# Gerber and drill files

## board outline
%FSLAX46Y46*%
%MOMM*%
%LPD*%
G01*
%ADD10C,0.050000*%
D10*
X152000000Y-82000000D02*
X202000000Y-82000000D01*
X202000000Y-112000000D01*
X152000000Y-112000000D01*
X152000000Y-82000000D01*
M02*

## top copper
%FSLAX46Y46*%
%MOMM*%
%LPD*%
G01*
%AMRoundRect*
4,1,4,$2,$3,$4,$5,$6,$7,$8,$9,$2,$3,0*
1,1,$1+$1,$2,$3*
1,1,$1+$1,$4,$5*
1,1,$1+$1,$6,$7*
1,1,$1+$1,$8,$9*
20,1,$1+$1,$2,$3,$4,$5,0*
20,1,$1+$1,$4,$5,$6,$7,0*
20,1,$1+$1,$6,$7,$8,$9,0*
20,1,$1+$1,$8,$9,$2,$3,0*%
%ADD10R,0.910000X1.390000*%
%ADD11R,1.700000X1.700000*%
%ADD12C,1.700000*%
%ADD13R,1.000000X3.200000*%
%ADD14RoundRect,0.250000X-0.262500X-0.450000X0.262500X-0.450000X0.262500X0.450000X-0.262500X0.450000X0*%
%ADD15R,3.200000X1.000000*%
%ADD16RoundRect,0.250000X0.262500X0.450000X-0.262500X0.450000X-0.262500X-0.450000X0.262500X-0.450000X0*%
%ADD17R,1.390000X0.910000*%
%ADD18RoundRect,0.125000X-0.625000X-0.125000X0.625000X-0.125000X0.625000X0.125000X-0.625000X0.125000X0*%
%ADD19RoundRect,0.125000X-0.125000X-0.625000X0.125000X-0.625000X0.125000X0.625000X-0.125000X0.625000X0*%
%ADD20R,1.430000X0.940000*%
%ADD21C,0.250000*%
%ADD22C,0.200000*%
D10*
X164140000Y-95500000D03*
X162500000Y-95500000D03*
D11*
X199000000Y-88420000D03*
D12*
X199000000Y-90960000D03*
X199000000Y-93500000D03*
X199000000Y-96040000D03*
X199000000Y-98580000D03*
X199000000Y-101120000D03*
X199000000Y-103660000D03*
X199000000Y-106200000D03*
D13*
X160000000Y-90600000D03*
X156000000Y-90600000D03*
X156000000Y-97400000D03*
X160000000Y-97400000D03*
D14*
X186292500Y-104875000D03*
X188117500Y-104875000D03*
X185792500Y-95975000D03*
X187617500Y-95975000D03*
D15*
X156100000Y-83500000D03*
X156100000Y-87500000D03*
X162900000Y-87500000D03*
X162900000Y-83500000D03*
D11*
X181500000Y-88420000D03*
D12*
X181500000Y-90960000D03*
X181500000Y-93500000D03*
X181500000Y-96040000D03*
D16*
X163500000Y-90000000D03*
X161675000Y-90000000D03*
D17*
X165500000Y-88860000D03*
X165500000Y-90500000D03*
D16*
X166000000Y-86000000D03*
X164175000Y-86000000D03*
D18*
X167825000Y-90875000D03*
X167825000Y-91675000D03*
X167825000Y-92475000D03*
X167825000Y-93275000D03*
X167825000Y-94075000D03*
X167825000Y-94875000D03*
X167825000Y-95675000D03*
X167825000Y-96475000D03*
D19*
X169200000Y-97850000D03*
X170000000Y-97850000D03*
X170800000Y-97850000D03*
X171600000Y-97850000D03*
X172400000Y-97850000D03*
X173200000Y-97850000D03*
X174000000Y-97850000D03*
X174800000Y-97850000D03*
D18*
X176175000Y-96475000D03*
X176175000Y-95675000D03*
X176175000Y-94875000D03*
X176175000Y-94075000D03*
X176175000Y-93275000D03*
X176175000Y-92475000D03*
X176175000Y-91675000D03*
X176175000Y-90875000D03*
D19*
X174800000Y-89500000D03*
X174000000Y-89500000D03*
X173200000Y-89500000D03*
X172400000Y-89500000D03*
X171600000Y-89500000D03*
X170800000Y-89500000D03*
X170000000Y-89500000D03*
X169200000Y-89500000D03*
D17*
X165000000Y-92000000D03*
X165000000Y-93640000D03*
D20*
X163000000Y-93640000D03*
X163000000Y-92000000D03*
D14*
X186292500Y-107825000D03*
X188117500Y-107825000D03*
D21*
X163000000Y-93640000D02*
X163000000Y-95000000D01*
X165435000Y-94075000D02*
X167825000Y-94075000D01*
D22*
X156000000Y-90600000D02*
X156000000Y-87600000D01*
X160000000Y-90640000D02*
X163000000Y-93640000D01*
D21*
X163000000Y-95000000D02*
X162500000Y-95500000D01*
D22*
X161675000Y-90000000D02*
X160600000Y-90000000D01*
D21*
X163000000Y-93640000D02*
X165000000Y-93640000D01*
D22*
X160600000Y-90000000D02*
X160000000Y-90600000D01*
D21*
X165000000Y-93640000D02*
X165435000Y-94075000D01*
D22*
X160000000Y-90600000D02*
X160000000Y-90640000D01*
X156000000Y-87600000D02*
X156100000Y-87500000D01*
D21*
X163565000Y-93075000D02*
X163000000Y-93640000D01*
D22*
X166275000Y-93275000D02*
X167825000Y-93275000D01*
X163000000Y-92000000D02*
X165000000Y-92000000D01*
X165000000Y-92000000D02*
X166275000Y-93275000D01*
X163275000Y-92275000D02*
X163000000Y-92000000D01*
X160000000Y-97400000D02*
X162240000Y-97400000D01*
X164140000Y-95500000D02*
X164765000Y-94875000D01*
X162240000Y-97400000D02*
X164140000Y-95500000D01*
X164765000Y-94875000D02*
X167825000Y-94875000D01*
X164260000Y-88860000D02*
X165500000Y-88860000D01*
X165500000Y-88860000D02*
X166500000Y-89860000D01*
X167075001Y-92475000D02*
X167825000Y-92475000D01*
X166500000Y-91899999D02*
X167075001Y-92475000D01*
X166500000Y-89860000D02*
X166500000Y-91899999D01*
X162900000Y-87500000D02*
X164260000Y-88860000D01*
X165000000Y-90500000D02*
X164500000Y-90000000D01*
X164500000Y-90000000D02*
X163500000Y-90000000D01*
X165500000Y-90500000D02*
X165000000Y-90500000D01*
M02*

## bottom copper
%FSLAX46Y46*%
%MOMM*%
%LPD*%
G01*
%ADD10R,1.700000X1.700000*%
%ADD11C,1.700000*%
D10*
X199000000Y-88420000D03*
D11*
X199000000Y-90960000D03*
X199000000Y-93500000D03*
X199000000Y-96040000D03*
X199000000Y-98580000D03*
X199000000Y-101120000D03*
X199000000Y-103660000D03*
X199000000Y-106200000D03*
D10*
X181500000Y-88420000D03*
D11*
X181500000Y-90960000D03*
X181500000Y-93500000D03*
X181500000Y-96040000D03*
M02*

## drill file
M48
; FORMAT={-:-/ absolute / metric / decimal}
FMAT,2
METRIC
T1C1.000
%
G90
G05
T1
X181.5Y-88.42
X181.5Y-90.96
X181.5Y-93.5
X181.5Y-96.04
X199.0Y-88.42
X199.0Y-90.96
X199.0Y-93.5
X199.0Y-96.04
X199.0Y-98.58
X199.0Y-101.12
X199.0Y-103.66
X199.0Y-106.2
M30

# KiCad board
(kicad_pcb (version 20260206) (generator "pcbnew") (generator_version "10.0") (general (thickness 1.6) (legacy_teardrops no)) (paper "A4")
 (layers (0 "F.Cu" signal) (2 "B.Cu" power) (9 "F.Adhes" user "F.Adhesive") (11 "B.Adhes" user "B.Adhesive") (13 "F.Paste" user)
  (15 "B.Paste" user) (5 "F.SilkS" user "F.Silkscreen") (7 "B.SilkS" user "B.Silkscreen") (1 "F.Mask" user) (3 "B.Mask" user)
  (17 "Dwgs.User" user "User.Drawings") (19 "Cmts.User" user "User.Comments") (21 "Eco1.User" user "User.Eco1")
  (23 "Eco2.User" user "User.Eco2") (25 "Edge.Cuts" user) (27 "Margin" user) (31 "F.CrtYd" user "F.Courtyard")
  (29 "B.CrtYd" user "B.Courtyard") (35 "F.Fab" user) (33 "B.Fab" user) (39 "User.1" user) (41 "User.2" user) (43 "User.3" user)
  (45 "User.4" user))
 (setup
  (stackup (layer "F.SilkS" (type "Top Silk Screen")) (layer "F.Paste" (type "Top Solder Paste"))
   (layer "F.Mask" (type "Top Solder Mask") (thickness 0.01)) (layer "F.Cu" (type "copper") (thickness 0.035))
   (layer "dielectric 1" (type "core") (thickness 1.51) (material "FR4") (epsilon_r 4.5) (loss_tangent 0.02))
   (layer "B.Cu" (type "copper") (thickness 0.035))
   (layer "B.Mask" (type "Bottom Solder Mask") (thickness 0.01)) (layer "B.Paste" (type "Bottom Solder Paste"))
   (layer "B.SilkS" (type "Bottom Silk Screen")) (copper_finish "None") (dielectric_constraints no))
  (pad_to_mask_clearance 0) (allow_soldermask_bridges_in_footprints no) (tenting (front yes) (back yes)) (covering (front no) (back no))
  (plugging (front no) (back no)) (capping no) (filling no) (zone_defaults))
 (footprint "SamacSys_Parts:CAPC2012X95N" (layer "F.Cu") (at 163.32 95.5 180)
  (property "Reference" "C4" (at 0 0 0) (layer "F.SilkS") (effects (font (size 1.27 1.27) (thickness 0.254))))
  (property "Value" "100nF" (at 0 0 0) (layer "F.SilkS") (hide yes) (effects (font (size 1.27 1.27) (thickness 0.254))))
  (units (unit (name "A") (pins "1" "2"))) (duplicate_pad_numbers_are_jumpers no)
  (pad "1" smd rect (at -0.82 0 180) (size 0.91 1.39) (layers "F.Cu" "F.Mask" "F.Paste") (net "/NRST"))
  (pad "2" smd rect (at 0.82 0 180) (size 0.91 1.39) (layers "F.Cu" "F.Mask" "F.Paste") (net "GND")))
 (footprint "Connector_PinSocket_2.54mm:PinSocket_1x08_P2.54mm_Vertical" (layer "F.Cu") (at 199 88.42)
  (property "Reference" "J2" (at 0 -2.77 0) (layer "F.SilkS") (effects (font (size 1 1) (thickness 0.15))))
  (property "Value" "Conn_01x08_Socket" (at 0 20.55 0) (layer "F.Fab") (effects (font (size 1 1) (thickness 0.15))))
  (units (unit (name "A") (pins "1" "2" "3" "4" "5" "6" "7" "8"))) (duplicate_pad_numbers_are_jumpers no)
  (pad "1" thru_hole rect (at 0 0) (size 1.7 1.7) (drill 1) (layers "*.Cu" "*.Mask") (remove_unused_layers no) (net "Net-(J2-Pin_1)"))
  (pad "2" thru_hole circle (at 0 2.54) (size 1.7 1.7) (drill 1) (layers "*.Cu" "*.Mask") (remove_unused_layers no)
   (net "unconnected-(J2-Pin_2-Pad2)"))
  (pad "3" thru_hole circle (at 0 5.08) (size 1.7 1.7) (drill 1) (layers "*.Cu" "*.Mask") (remove_unused_layers no)
   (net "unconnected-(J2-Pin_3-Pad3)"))
  (pad "4" thru_hole circle (at 0 7.62) (size 1.7 1.7) (drill 1) (layers "*.Cu" "*.Mask") (remove_unused_layers no)
   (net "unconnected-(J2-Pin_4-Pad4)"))
  (pad "5" thru_hole circle (at 0 10.16) (size 1.7 1.7) (drill 1) (layers "*.Cu" "*.Mask") (remove_unused_layers no)
   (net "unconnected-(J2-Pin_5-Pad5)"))
  (pad "6" thru_hole circle (at 0 12.7) (size 1.7 1.7) (drill 1) (layers "*.Cu" "*.Mask") (remove_unused_layers no)
   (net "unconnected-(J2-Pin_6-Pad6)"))
  (pad "7" thru_hole circle (at 0 15.24) (size 1.7 1.7) (drill 1) (layers "*.Cu" "*.Mask") (remove_unused_layers no)
   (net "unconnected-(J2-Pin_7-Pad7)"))
  (pad "8" thru_hole circle (at 0 17.78) (size 1.7 1.7) (drill 1) (layers "*.Cu" "*.Mask") (remove_unused_layers no)
   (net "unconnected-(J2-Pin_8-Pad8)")))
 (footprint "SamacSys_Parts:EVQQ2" (layer "F.Cu") (at 158 94 -90)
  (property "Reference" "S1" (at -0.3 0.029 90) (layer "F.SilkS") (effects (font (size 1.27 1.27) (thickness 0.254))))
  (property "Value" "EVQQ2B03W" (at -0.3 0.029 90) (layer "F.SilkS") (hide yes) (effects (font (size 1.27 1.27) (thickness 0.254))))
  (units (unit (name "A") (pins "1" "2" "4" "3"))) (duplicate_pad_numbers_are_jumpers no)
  (pad "1" smd rect (at -3.4 -2) (size 1 3.2) (layers "F.Cu" "F.Mask" "F.Paste") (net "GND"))
  (pad "2" smd rect (at -3.4 2) (size 1 3.2) (layers "F.Cu" "F.Mask" "F.Paste") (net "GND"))
  (pad "3" smd rect (at 3.4 2) (size 1 3.2) (layers "F.Cu" "F.Mask" "F.Paste") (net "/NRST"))
  (pad "4" smd rect (at 3.4 -2) (size 1 3.2) (layers "F.Cu" "F.Mask" "F.Paste") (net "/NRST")))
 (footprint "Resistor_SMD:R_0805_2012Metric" (layer "F.Cu") (at 187.205 104.875)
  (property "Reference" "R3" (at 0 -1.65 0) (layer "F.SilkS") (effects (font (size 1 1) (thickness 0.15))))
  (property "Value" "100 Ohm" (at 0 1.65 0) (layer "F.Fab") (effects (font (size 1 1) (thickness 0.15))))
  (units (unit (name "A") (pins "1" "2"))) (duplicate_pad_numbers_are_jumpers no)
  (pad "1" smd roundrect (at -0.9125 0) (size 1.025 1.4) (layers "F.Cu" "F.Mask" "F.Paste") (roundrect_rratio 0.243902)
   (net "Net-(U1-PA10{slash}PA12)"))
  (pad "2" smd roundrect (at 0.9125 0) (size 1.025 1.4) (layers "F.Cu" "F.Mask" "F.Paste") (roundrect_rratio 0.243902)
   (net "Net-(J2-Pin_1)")))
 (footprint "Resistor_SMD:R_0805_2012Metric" (layer "F.Cu") (at 186.705 95.975)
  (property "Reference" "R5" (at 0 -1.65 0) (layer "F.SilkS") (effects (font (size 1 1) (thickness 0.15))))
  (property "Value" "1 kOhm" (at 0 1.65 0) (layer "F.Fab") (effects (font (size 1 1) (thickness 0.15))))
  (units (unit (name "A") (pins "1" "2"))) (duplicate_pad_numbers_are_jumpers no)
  (pad "1" smd roundrect (at -0.9125 0) (size 1.025 1.4) (layers "F.Cu" "F.Mask" "F.Paste") (roundrect_rratio 0.243902) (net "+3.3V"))
  (pad "2" smd roundrect (at 0.9125 0) (size 1.025 1.4) (layers "F.Cu" "F.Mask" "F.Paste") (roundrect_rratio 0.243902)
   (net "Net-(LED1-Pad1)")))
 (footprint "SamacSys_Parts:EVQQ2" (layer "F.Cu") (at 159.5 85.5)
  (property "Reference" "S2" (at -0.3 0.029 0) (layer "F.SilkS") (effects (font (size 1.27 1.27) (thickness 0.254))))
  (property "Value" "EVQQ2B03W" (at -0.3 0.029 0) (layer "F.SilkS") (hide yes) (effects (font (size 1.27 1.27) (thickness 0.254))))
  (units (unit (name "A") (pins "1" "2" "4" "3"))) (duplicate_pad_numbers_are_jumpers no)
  (pad "1" smd rect (at -3.4 -2 90) (size 1 3.2) (layers "F.Cu" "F.Mask" "F.Paste") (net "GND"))
  (pad "2" smd rect (at -3.4 2 90) (size 1 3.2) (layers "F.Cu" "F.Mask" "F.Paste") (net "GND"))
  (pad "3" smd rect (at 3.4 2 90) (size 1 3.2) (layers "F.Cu" "F.Mask" "F.Paste") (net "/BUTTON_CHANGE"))
  (pad "4" smd rect (at 3.4 -2 90) (size 1 3.2) (layers "F.Cu" "F.Mask" "F.Paste") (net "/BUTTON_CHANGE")))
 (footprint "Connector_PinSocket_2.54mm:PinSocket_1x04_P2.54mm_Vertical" (layer "F.Cu") (at 181.5 88.42)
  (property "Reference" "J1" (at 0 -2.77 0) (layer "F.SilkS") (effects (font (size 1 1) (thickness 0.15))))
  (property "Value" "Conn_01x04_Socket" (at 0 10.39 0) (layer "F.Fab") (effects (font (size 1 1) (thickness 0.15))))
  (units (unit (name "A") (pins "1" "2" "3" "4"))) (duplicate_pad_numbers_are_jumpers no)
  (pad "1" thru_hole rect (at 0 0) (size 1.7 1.7) (drill 1) (layers "*.Cu" "*.Mask") (remove_unused_layers no)
   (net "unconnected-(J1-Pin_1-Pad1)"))
  (pad "2" thru_hole circle (at 0 2.54) (size 1.7 1.7) (drill 1) (layers "*.Cu" "*.Mask") (remove_unused_layers no)
   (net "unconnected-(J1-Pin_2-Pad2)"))
  (pad "3" thru_hole circle (at 0 5.08) (size 1.7 1.7) (drill 1) (layers "*.Cu" "*.Mask") (remove_unused_layers no)
   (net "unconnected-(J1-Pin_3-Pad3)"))
  (pad "4" thru_hole circle (at 0 7.62) (size 1.7 1.7) (drill 1) (layers "*.Cu" "*.Mask") (remove_unused_layers no)
   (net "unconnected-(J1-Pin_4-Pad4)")))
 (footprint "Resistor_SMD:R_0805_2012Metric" (layer "F.Cu") (at 162.5875 90 180)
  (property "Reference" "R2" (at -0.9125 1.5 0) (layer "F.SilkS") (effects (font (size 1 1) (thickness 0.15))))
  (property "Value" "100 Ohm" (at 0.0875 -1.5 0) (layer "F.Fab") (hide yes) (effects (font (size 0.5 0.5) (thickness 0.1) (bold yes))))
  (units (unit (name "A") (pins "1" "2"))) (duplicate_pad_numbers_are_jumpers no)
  (pad "1" smd roundrect (at -0.9125 0 180) (size 1.025 1.4) (layers "F.Cu" "F.Mask" "F.Paste") (roundrect_rratio 0.243902)
   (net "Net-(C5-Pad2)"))
  (pad "2" smd roundrect (at 0.9125 0 180) (size 1.025 1.4) (layers "F.Cu" "F.Mask" "F.Paste") (roundrect_rratio 0.243902) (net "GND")))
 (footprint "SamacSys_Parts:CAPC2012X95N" (layer "F.Cu") (at 165.5 89.68 -90)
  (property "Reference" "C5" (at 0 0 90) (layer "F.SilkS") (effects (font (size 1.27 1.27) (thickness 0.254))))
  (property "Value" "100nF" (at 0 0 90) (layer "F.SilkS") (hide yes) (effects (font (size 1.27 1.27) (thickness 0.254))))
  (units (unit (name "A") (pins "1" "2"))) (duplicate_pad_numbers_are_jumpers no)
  (pad "1" smd rect (at -0.82 0 270) (size 0.91 1.39) (layers "F.Cu" "F.Mask" "F.Paste") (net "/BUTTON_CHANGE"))
  (pad "2" smd rect (at 0.82 0 270) (size 0.91 1.39) (layers "F.Cu" "F.Mask" "F.Paste") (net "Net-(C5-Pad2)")))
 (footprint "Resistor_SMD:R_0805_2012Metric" (layer "F.Cu") (at 165.0875 86 180)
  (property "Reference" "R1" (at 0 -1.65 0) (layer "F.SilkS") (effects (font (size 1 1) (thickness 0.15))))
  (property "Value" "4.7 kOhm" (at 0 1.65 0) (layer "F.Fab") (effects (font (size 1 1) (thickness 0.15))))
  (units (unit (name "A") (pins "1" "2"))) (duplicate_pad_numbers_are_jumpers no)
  (pad "1" smd roundrect (at -0.9125 0 180) (size 1.025 1.4) (layers "F.Cu" "F.Mask" "F.Paste") (roundrect_rratio 0.243902) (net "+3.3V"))
  (pad "2" smd roundrect (at 0.9125 0 180) (size 1.025 1.4) (layers "F.Cu" "F.Mask" "F.Paste") (roundrect_rratio 0.243902)
   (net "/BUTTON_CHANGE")))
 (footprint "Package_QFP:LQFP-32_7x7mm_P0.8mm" (layer "F.Cu") (at 172 93.675)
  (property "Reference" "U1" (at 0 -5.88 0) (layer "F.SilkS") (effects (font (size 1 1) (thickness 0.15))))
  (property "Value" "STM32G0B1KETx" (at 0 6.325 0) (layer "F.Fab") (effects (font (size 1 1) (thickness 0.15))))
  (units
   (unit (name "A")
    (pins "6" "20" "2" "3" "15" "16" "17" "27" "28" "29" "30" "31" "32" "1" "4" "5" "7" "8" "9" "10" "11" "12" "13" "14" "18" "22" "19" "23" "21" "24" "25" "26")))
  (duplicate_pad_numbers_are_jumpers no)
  (pad "1" smd roundrect (at -4.175 -2.8) (size 1.5 0.5) (layers "F.Cu" "F.Mask" "F.Paste") (roundrect_rratio 0.25)
   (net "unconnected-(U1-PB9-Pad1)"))
  (pad "2" smd roundrect (at -4.175 -2) (size 1.5 0.5) (layers "F.Cu" "F.Mask" "F.Paste") (roundrect_rratio 0.25)
   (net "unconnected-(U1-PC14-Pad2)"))
  (pad "3" smd roundrect (at -4.175 -1.2) (size 1.5 0.5) (layers "F.Cu" "F.Mask" "F.Paste") (roundrect_rratio 0.25) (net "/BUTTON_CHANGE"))
  (pad "4" smd roundrect (at -4.175 -0.4) (size 1.5 0.5) (layers "F.Cu" "F.Mask" "F.Paste") (roundrect_rratio 0.25) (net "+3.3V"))
  (pad "5" smd roundrect (at -4.175 0.4) (size 1.5 0.5) (layers "F.Cu" "F.Mask" "F.Paste") (roundrect_rratio 0.25) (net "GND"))
  (pad "6" smd roundrect (at -4.175 1.2) (size 1.5 0.5) (layers "F.Cu" "F.Mask" "F.Paste") (roundrect_rratio 0.25) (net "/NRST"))
  (pad "7" smd roundrect (at -4.175 2) (size 1.5 0.5) (layers "F.Cu" "F.Mask" "F.Paste") (roundrect_rratio 0.25)
   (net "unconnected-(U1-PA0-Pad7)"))
  (pad "8" smd roundrect (at -4.175 2.8) (size 1.5 0.5) (layers "F.Cu" "F.Mask" "F.Paste") (roundrect_rratio 0.25)
   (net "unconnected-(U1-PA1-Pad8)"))
  (pad "9" smd roundrect (at -2.8 4.175) (size 0.5 1.5) (layers "F.Cu" "F.Mask" "F.Paste") (roundrect_rratio 0.25)
   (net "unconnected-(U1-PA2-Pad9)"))
  (pad "10" smd roundrect (at -2 4.175) (size 0.5 1.5) (layers "F.Cu" "F.Mask" "F.Paste") (roundrect_rratio 0.25)
   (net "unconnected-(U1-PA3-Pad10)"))
  (pad "11" smd roundrect (at -1.2 4.175) (size 0.5 1.5) (layers "F.Cu" "F.Mask" "F.Paste") (roundrect_rratio 0.25)
   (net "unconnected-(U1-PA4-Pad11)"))
  (pad "12" smd roundrect (at -0.4 4.175) (size 0.5 1.5) (layers "F.Cu" "F.Mask" "F.Paste") (roundrect_rratio 0.25)
   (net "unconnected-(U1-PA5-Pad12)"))
  (pad "13" smd roundrect (at 0.4 4.175) (size 0.5 1.5) (layers "F.Cu" "F.Mask" "F.Paste") (roundrect_rratio 0.25)
   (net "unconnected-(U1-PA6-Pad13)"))
  (pad "14" smd roundrect (at 1.2 4.175) (size 0.5 1.5) (layers "F.Cu" "F.Mask" "F.Paste") (roundrect_rratio 0.25)
   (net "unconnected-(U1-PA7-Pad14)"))
  (pad "15" smd roundrect (at 2 4.175) (size 0.5 1.5) (layers "F.Cu" "F.Mask" "F.Paste") (roundrect_rratio 0.25)
   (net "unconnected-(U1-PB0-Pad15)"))
  (pad "16" smd roundrect (at 2.8 4.175) (size 0.5 1.5) (layers "F.Cu" "F.Mask" "F.Paste") (roundrect_rratio 0.25)
   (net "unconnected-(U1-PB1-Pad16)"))
  (pad "17" smd roundrect (at 4.175 2.8) (size 1.5 0.5) (layers "F.Cu" "F.Mask" "F.Paste") (roundrect_rratio 0.25)
   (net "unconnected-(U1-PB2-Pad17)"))
  (pad "18" smd roundrect (at 4.175 2) (size 1.5 0.5) (layers "F.Cu" "F.Mask" "F.Paste") (roundrect_rratio 0.25)
   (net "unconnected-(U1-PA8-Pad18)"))
  (pad "19" smd roundrect (at 4.175 1.2) (size 1.5 0.5) (layers "F.Cu" "F.Mask" "F.Paste") (roundrect_rratio 0.25)
   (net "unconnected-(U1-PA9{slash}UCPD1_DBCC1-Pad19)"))
  (pad "20" smd roundrect (at 4.175 0.4) (size 1.5 0.5) (layers "F.Cu" "F.Mask" "F.Paste") (roundrect_rratio 0.25)
   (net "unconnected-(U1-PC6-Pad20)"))
  (pad "21" smd roundrect (at 4.175 -0.4) (size 1.5 0.5) (layers "F.Cu" "F.Mask" "F.Paste") (roundrect_rratio 0.25)
   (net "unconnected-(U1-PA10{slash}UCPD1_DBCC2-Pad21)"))
  (pad "22" smd roundrect (at 4.175 -1.2) (size 1.5 0.5) (layers "F.Cu" "F.Mask" "F.Paste") (roundrect_rratio 0.25)
   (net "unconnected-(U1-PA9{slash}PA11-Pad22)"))
  (pad "23" smd roundrect (at 4.175 -2) (size 1.5 0.5) (layers "F.Cu" "F.Mask" "F.Paste") (roundrect_rratio 0.25)
   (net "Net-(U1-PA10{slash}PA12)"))
  (pad "24" smd roundrect (at 4.175 -2.8) (size 1.5 0.5) (layers "F.Cu" "F.Mask" "F.Paste") (roundrect_rratio 0.25)
   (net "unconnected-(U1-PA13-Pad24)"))
  (pad "25" smd roundrect (at 2.8 -4.175) (size 0.5 1.5) (layers "F.Cu" "F.Mask" "F.Paste") (roundrect_rratio 0.25)
   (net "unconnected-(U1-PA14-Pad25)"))
  (pad "26" smd roundrect (at 2 -4.175) (size 0.5 1.5) (layers "F.Cu" "F.Mask" "F.Paste") (roundrect_rratio 0.25)
   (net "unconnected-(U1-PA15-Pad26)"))
  (pad "27" smd roundrect (at 1.2 -4.175) (size 0.5 1.5) (layers "F.Cu" "F.Mask" "F.Paste") (roundrect_rratio 0.25)
   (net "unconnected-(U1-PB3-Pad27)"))
  (pad "28" smd roundrect (at 0.4 -4.175) (size 0.5 1.5) (layers "F.Cu" "F.Mask" "F.Paste") (roundrect_rratio 0.25)
   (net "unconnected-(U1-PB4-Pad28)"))
  (pad "29" smd roundrect (at -0.4 -4.175) (size 0.5 1.5) (layers "F.Cu" "F.Mask" "F.Paste") (roundrect_rratio 0.25)
   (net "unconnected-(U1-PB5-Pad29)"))
  (pad "30" smd roundrect (at -1.2 -4.175) (size 0.5 1.5) (layers "F.Cu" "F.Mask" "F.Paste") (roundrect_rratio 0.25)
   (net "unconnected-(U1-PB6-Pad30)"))
  (pad "31" smd roundrect (at -2 -4.175) (size 0.5 1.5) (layers "F.Cu" "F.Mask" "F.Paste") (roundrect_rratio 0.25)
   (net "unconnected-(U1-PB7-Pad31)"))
  (pad "32" smd roundrect (at -2.8 -4.175) (size 0.5 1.5) (layers "F.Cu" "F.Mask" "F.Paste") (roundrect_rratio 0.25)
   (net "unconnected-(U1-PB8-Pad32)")))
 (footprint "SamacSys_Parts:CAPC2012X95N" (layer "F.Cu") (at 165 92.82 -90)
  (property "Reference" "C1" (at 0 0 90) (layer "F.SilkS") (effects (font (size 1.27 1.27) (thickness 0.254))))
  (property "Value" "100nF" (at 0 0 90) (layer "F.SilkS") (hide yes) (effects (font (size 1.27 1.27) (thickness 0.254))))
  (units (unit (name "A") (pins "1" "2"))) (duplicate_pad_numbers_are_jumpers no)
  (pad "1" smd rect (at -0.82 0 270) (size 0.91 1.39) (layers "F.Cu" "F.Mask" "F.Paste") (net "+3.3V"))
  (pad "2" smd rect (at 0.82 0 270) (size 0.91 1.39) (layers "F.Cu" "F.Mask" "F.Paste") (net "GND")))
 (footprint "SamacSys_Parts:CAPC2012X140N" (layer "F.Cu") (at 163 92.82 90)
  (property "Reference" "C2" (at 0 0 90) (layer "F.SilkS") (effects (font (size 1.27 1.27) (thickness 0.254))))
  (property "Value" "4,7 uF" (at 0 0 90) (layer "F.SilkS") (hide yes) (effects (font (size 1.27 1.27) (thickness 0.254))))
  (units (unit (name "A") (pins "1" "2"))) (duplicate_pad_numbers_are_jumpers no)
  (pad "1" smd rect (at -0.82 0 90) (size 0.94 1.43) (layers "F.Cu" "F.Mask" "F.Paste") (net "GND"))
  (pad "2" smd rect (at 0.82 0 90) (size 0.94 1.43) (layers "F.Cu" "F.Mask" "F.Paste") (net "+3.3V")))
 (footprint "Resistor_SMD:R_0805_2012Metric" (layer "F.Cu") (at 187.205 107.825)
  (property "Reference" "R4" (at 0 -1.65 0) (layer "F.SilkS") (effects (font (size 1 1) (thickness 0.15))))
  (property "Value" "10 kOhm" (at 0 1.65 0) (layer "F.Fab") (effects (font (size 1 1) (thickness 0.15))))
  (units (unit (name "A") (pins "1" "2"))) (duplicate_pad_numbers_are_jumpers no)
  (pad "1" smd roundrect (at -0.9125 0) (size 1.025 1.4) (layers "F.Cu" "F.Mask" "F.Paste") (roundrect_rratio 0.243902) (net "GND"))
  (pad "2" smd roundrect (at 0.9125 0) (size 1.025 1.4) (layers "F.Cu" "F.Mask" "F.Paste") (roundrect_rratio 0.243902)
   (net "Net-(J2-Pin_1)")))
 (gr_rect (start 152 82) (end 202 112) (stroke (width 0.05) (type default)) (fill no) (layer "Edge.Cuts"))
 (segment (start 163 93.64) (end 163 95) (width 0.25) (layer "F.Cu") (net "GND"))
 (segment (start 165.435 94.075) (end 167.825 94.075) (width 0.25) (layer "F.Cu") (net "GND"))
 (segment (start 156 90.6) (end 156 87.6) (width 0.2) (layer "F.Cu") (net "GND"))
 (segment (start 160 90.64) (end 163 93.64) (width 0.2) (layer "F.Cu") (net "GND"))
 (segment (start 163 95) (end 162.5 95.5) (width 0.25) (layer "F.Cu") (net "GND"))
 (segment (start 161.675 90) (end 160.6 90) (width 0.2) (layer "F.Cu") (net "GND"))
 (segment (start 163 93.64) (end 165 93.64) (width 0.25) (layer "F.Cu") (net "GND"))
 (segment (start 160.6 90) (end 160 90.6) (width 0.2) (layer "F.Cu") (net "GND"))
 (segment (start 165 93.64) (end 165.435 94.075) (width 0.25) (layer "F.Cu") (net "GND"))
 (segment (start 160 90.6) (end 160 90.64) (width 0.2) (layer "F.Cu") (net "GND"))
 (segment (start 156 87.6) (end 156.1 87.5) (width 0.2) (layer "F.Cu") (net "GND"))
 (segment (start 163.565 93.075) (end 163 93.64) (width 0.25) (layer "F.Cu") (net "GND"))
 (segment (start 166.275 93.275) (end 167.825 93.275) (width 0.2) (layer "F.Cu") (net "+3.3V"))
 (segment (start 163 92) (end 165 92) (width 0.2) (layer "F.Cu") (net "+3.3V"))
 (segment (start 165 92) (end 166.275 93.275) (width 0.2) (layer "F.Cu") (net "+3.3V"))
 (segment (start 163.275 92.275) (end 163 92) (width 0.2) (layer "F.Cu") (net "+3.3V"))
 (segment (start 160 97.4) (end 162.24 97.4) (width 0.2) (layer "F.Cu") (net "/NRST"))
 (segment (start 164.14 95.5) (end 164.765 94.875) (width 0.2) (layer "F.Cu") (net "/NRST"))
 (segment (start 162.24 97.4) (end 164.14 95.5) (width 0.2) (layer "F.Cu") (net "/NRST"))
 (segment (start 164.765 94.875) (end 167.825 94.875) (width 0.2) (layer "F.Cu") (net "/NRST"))
 (segment (start 164.26 88.86) (end 165.5 88.86) (width 0.2) (layer "F.Cu") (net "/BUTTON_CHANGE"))
 (segment (start 165.5 88.86) (end 166.5 89.86) (width 0.2) (layer "F.Cu") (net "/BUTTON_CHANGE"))
 (segment (start 167.075001 92.475) (end 167.825 92.475) (width 0.2) (layer "F.Cu") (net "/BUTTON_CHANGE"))
 (segment (start 166.5 91.899999) (end 167.075001 92.475) (width 0.2) (layer "F.Cu") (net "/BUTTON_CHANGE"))
 (segment (start 166.5 89.86) (end 166.5 91.899999) (width 0.2) (layer "F.Cu") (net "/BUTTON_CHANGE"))
 (segment (start 162.9 87.5) (end 164.26 88.86) (width 0.2) (layer "F.Cu") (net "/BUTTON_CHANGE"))
 (segment (start 165 90.5) (end 164.5 90) (width 0.2) (layer "F.Cu") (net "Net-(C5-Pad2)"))
 (segment (start 164.5 90) (end 163.5 90) (width 0.2) (layer "F.Cu") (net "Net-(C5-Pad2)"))
 (segment (start 165.5 90.5) (end 165 90.5) (width 0.2) (layer "F.Cu") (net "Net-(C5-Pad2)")))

